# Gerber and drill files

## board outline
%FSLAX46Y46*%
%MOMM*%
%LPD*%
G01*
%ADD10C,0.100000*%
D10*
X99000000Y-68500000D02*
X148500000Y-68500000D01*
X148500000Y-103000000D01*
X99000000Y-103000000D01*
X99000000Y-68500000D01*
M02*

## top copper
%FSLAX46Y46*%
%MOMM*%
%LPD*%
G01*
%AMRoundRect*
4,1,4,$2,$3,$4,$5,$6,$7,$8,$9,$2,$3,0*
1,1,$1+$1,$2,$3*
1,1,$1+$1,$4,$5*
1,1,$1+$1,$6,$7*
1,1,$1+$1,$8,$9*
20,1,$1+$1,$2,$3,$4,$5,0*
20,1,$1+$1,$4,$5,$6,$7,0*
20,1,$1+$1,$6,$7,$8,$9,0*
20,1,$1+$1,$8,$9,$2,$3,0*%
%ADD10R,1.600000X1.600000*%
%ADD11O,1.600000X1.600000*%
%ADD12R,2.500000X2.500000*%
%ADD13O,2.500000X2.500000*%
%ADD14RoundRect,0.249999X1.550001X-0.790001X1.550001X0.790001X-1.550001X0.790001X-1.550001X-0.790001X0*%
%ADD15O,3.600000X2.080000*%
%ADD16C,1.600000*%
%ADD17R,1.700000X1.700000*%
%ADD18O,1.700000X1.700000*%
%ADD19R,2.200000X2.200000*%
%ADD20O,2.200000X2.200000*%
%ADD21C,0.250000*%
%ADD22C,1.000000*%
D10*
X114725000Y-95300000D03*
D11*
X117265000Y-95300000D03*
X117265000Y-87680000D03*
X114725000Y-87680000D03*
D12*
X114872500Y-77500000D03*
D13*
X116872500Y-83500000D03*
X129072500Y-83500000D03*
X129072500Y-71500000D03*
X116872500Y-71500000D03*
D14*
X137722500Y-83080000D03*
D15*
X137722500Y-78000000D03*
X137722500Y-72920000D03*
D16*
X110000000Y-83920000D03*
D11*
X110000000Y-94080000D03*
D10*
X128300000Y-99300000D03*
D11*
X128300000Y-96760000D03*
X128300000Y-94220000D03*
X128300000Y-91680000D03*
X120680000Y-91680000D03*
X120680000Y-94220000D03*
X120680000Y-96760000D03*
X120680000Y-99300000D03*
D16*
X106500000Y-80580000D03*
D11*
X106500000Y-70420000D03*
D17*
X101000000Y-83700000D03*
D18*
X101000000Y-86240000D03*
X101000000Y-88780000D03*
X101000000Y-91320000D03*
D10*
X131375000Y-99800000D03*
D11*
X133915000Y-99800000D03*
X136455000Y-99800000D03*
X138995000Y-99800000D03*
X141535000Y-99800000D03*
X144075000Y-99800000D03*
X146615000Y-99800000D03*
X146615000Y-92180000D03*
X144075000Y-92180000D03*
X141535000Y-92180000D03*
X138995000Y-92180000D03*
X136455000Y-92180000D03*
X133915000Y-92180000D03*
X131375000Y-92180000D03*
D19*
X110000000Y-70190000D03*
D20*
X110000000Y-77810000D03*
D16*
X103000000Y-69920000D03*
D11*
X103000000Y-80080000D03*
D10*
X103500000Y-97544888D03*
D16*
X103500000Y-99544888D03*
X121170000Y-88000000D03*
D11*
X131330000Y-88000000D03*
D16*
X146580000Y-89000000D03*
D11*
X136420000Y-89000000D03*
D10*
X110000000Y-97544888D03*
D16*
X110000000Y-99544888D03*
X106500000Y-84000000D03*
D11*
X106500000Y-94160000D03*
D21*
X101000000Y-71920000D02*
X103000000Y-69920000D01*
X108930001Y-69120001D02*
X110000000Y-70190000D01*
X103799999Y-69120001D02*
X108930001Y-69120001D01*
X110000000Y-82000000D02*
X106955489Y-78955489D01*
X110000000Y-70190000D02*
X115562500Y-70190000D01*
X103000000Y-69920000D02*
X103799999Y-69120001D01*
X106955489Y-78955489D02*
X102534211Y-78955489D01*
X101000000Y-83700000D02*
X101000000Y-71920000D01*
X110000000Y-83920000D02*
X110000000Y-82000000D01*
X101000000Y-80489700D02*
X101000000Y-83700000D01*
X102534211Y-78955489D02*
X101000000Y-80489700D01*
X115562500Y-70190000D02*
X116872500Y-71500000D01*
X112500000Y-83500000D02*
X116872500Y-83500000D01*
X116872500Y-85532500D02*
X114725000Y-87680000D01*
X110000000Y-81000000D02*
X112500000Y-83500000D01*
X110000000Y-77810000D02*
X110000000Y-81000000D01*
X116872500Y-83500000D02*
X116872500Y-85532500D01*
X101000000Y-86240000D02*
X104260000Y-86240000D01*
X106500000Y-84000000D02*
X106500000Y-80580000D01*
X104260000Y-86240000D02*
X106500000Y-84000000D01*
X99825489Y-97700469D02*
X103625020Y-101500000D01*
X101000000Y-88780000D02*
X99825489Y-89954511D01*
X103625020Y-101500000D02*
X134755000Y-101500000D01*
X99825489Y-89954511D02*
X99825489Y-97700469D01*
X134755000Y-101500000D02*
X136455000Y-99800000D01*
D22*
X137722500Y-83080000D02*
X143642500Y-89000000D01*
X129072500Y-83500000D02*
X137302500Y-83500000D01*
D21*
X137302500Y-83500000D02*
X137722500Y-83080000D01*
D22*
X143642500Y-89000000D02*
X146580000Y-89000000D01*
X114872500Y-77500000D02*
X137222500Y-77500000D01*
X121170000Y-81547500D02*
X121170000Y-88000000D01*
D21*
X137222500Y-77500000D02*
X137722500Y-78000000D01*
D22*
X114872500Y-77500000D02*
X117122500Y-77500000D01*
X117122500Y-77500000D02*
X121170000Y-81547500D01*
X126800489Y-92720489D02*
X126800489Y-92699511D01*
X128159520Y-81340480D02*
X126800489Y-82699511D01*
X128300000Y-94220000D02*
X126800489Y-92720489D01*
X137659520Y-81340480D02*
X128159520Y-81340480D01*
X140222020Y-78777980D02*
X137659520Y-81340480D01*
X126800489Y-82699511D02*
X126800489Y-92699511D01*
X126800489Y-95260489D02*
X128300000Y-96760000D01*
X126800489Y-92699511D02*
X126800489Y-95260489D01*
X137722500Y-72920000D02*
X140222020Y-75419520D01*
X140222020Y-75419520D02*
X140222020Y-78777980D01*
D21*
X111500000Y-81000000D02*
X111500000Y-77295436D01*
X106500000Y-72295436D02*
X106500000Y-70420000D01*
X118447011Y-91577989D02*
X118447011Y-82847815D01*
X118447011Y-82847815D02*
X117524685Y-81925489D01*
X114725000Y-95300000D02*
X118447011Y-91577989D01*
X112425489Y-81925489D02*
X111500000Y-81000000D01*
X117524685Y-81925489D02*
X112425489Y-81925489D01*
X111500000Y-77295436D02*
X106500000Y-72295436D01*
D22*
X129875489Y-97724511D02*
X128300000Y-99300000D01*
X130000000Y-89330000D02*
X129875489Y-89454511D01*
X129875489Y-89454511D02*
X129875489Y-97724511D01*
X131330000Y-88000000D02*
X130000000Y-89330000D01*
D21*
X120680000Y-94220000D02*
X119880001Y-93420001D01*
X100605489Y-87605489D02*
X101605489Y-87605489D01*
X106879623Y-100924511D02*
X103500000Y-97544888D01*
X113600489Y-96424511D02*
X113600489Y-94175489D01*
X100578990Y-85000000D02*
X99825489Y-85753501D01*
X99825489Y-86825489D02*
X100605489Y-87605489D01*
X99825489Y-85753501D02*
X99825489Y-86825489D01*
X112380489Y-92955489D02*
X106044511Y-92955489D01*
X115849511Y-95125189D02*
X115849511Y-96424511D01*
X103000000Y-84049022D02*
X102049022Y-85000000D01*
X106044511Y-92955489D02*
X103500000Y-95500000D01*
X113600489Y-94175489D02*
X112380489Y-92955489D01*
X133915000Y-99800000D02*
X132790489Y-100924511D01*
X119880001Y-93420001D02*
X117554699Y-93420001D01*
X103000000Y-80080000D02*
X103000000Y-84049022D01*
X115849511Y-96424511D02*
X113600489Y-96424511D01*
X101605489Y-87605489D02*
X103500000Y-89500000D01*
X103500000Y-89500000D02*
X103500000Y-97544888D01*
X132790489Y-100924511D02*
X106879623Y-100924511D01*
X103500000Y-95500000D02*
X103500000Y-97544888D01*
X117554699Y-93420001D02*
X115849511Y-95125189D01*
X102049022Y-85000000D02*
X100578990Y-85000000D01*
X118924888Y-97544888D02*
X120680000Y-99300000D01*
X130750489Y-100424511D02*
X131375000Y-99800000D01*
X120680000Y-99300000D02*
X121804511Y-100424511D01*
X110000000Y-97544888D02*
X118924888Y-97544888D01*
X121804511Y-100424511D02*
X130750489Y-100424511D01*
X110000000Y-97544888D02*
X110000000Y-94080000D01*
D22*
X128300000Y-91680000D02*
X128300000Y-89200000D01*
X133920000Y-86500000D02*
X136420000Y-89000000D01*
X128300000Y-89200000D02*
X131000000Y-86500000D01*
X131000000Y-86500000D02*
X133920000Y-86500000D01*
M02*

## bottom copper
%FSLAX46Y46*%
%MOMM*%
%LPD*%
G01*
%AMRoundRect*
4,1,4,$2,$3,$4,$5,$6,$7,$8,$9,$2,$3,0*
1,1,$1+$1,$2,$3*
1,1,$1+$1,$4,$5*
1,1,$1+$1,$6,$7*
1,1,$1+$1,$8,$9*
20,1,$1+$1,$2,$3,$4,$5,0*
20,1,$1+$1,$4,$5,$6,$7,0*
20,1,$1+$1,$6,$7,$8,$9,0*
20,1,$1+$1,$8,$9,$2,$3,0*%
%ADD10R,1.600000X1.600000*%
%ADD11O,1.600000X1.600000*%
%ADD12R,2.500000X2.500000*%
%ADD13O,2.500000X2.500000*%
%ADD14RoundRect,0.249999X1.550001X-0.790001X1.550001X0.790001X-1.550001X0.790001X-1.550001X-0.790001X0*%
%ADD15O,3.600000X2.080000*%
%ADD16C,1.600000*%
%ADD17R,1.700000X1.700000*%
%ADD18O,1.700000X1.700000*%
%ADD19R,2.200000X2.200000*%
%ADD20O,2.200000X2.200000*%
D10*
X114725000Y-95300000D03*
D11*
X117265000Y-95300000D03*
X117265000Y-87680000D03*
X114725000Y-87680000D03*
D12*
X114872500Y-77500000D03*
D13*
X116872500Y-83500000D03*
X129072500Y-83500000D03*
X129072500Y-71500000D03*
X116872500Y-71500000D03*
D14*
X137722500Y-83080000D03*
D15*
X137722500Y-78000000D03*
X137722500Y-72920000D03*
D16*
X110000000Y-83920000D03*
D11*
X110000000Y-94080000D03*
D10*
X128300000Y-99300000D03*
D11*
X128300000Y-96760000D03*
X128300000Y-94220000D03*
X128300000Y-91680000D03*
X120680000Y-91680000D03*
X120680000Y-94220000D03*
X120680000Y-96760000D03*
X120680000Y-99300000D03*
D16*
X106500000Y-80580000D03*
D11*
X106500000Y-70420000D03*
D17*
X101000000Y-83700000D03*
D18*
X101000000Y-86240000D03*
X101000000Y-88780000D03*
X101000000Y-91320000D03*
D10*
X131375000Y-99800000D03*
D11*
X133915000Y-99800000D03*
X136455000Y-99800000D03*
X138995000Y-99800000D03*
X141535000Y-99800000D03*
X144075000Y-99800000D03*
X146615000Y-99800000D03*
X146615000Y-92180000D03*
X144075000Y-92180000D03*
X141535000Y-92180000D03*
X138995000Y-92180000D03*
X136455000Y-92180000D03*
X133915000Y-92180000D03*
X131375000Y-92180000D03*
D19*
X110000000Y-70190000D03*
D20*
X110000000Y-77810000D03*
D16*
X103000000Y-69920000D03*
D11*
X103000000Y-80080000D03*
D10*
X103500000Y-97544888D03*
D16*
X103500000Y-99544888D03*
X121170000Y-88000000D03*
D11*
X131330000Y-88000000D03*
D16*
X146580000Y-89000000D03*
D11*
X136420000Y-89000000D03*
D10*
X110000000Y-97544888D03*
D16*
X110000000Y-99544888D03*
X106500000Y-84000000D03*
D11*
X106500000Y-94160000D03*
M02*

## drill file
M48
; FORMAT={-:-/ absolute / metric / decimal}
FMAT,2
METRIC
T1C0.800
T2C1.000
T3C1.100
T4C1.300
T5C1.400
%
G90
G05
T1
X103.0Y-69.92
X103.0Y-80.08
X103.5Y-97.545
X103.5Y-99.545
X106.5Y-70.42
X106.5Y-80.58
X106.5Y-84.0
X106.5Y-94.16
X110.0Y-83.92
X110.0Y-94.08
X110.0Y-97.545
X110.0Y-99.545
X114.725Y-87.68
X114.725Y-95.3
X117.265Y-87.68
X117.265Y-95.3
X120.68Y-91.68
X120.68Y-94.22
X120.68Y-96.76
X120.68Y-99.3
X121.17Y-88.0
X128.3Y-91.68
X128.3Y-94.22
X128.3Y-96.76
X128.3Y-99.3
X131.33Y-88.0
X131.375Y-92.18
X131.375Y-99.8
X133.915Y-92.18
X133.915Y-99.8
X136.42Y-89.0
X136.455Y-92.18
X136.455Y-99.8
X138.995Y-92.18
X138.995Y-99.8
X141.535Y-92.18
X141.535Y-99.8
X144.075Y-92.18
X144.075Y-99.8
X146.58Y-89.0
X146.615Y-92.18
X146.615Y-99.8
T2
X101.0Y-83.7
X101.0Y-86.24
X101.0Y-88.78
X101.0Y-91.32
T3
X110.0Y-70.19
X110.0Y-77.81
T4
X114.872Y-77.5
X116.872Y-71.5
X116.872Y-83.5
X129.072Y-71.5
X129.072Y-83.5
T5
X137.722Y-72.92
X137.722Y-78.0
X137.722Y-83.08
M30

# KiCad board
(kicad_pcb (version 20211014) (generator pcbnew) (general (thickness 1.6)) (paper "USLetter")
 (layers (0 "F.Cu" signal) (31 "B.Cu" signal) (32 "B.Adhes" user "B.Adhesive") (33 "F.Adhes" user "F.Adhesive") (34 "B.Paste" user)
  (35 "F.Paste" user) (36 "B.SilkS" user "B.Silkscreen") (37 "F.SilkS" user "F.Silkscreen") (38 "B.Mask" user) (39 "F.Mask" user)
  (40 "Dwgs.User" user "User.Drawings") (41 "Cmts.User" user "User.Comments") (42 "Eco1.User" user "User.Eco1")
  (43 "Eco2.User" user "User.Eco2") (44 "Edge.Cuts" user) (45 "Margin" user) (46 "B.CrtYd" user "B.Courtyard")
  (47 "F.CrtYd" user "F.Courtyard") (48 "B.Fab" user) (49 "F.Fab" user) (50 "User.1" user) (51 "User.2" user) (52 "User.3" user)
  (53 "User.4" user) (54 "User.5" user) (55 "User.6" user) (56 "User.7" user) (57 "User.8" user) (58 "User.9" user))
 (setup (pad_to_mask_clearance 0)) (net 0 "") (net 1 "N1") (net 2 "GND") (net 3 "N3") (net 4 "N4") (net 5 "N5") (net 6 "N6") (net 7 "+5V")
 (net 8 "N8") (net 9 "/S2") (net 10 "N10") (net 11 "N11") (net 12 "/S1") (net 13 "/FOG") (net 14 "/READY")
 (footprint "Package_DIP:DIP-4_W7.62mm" (layer "F.Cu") (at 114.725 95.3 90)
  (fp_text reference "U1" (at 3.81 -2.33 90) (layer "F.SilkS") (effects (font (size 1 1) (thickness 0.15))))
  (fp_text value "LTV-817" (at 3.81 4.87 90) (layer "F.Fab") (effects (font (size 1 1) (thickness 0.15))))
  (pad "1" thru_hole rect locked (at 0 0 90) (size 1.6 1.6) (drill 0.8) (layers *.Cu *.Mask) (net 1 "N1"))
  (pad "2" thru_hole oval locked (at 0 2.54 90) (size 1.6 1.6) (drill 0.8) (layers *.Cu *.Mask) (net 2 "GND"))
  (pad "3" thru_hole oval locked (at 7.62 2.54 90) (size 1.6 1.6) (drill 0.8) (layers *.Cu *.Mask) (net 2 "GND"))
  (pad "4" thru_hole oval locked (at 7.62 0 90) (size 1.6 1.6) (drill 0.8) (layers *.Cu *.Mask) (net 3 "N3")))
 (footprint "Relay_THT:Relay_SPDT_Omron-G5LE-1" (layer "F.Cu") (at 114.8725 77.5 90)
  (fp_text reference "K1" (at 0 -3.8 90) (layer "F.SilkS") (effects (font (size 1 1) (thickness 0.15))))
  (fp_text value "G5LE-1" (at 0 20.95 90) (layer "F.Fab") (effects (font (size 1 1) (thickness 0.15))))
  (pad "1" thru_hole rect locked (at 0 0 90) (size 2.5 2.5) (drill 1.3) (layers *.Cu *.Mask) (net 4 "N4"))
  (pad "2" thru_hole oval locked (at -6 2 90) (size 2.5 2.5) (drill 1.3) (layers *.Cu *.Mask) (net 3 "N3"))
  (pad "3" thru_hole oval locked (at -6 14.2 90) (size 2.5 2.5) (drill 1.3) (layers *.Cu *.Mask) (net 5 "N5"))
  (pad "4" thru_hole oval locked (at 6 14.2 90) (size 2.5 2.5) (drill 1.3) (layers *.Cu *.Mask) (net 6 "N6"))
  (pad "5" thru_hole oval locked (at 6 2 90) (size 2.5 2.5) (drill 1.3) (layers *.Cu *.Mask) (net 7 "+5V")))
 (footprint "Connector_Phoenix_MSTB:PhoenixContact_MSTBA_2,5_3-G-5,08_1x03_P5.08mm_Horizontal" (layer "F.Cu") (at 137.7225 83.08 90)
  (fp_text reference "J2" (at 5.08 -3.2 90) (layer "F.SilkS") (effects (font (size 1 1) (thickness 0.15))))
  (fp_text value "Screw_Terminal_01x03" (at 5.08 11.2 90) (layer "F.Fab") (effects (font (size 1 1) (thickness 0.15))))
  (pad "1" thru_hole roundrect locked (at 0 0 90) (size 2.08 3.6) (drill 1.4) (layers *.Cu *.Mask) (roundrect_rratio 0.120192) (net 5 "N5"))
  (pad "2" thru_hole oval locked (at 5.08 0 90) (size 2.08 3.6) (drill 1.4) (layers *.Cu *.Mask) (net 4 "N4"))
  (pad "3" thru_hole oval locked (at 10.16 0 90) (size 2.08 3.6) (drill 1.4) (layers *.Cu *.Mask) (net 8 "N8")))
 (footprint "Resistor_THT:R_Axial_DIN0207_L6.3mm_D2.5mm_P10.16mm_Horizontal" (layer "F.Cu") (at 110 83.92 -90)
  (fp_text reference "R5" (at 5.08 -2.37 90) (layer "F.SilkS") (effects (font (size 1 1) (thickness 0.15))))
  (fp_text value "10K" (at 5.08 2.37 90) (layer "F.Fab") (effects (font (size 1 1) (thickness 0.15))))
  (pad "1" thru_hole circle locked (at 0 0 270) (size 1.6 1.6) (drill 0.8) (layers *.Cu *.Mask) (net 7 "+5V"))
  (pad "2" thru_hole oval locked (at 10.16 0 270) (size 1.6 1.6) (drill 0.8) (layers *.Cu *.Mask) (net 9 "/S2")))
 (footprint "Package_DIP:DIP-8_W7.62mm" (layer "F.Cu") (at 128.3 99.3 180)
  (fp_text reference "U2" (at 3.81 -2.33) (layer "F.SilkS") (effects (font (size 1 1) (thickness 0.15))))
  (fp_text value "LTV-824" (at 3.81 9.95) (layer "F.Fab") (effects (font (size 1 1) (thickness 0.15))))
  (pad "1" thru_hole rect locked (at 0 0 180) (size 1.6 1.6) (drill 0.8) (layers *.Cu *.Mask) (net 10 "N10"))
  (pad "2" thru_hole oval locked (at 0 2.54 180) (size 1.6 1.6) (drill 0.8) (layers *.Cu *.Mask) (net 8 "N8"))
  (pad "3" thru_hole oval locked (at 0 5.08 180) (size 1.6 1.6) (drill 0.8) (layers *.Cu *.Mask) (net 8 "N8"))
  (pad "4" thru_hole oval locked (at 0 7.62 180) (size 1.6 1.6) (drill 0.8) (layers *.Cu *.Mask) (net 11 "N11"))
  (pad "5" thru_hole oval locked (at 7.62 7.62 180) (size 1.6 1.6) (drill 0.8) (layers *.Cu *.Mask) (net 2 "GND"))
  (pad "6" thru_hole oval locked (at 7.62 5.08 180) (size 1.6 1.6) (drill 0.8) (layers *.Cu *.Mask) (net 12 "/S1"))
  (pad "7" thru_hole oval locked (at 7.62 2.54 180) (size 1.6 1.6) (drill 0.8) (layers *.Cu *.Mask) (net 2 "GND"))
  (pad "8" thru_hole oval locked (at 7.62 0 180) (size 1.6 1.6) (drill 0.8) (layers *.Cu *.Mask) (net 9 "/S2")))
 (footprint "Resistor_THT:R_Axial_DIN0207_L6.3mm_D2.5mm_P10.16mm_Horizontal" (layer "F.Cu") (at 106.5 80.58 90)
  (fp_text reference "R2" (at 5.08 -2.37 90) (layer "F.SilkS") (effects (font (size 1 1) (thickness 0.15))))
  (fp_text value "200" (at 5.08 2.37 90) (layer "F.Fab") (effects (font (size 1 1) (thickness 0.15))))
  (pad "1" thru_hole circle locked (at 0 0 90) (size 1.6 1.6) (drill 0.8) (layers *.Cu *.Mask) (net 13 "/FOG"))
  (pad "2" thru_hole oval locked (at 10.16 0 90) (size 1.6 1.6) (drill 0.8) (layers *.Cu *.Mask) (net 1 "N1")))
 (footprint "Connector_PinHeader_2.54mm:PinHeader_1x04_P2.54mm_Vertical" (layer "F.Cu") (at 101 83.7)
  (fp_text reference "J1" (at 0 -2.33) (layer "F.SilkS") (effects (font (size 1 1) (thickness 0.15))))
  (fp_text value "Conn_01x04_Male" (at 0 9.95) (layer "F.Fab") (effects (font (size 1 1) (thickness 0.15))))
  (pad "1" thru_hole rect locked (at 0 0) (size 1.7 1.7) (drill 1) (layers *.Cu *.Mask) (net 7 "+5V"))
  (pad "2" thru_hole oval locked (at 0 2.54) (size 1.7 1.7) (drill 1) (layers *.Cu *.Mask) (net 13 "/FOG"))
  (pad "3" thru_hole oval locked (at 0 5.08) (size 1.7 1.7) (drill 1) (layers *.Cu *.Mask) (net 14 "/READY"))
  (pad "4" thru_hole oval locked (at 0 7.62) (size 1.7 1.7) (drill 1) (layers *.Cu *.Mask) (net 2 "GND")))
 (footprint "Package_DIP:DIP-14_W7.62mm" (layer "F.Cu") (at 131.375 99.8 90)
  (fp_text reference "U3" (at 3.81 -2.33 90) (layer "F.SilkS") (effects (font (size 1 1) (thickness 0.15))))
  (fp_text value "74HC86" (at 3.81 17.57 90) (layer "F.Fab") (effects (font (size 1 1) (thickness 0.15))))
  (pad "1" thru_hole rect locked (at 0 0 90) (size 1.6 1.6) (drill 0.8) (layers *.Cu *.Mask) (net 9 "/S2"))
  (pad "2" thru_hole oval locked (at 0 2.54 90) (size 1.6 1.6) (drill 0.8) (layers *.Cu *.Mask) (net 12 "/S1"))
  (pad "3" thru_hole oval locked (at 0 5.08 90) (size 1.6 1.6) (drill 0.8) (layers *.Cu *.Mask) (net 14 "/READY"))
  (pad "4" thru_hole oval locked (at 0 7.62 90) (size 1.6 1.6) (drill 0.8) (layers *.Cu *.Mask))
  (pad "5" thru_hole oval locked (at 0 10.16 90) (size 1.6 1.6) (drill 0.8) (layers *.Cu *.Mask))
  (pad "6" thru_hole oval locked (at 0 12.7 90) (size 1.6 1.6) (drill 0.8) (layers *.Cu *.Mask))
  (pad "7" thru_hole oval locked (at 0 15.24 90) (size 1.6 1.6) (drill 0.8) (layers *.Cu *.Mask))
  (pad "8" thru_hole oval locked (at 7.62 15.24 90) (size 1.6 1.6) (drill 0.8) (layers *.Cu *.Mask))
  (pad "9" thru_hole oval locked (at 7.62 12.7 90) (size 1.6 1.6) (drill 0.8) (layers *.Cu *.Mask))
  (pad "10" thru_hole oval locked (at 7.62 10.16 90) (size 1.6 1.6) (drill 0.8) (layers *.Cu *.Mask))
  (pad "11" thru_hole oval locked (at 7.62 7.62 90) (size 1.6 1.6) (drill 0.8) (layers *.Cu *.Mask))
  (pad "12" thru_hole oval locked (at 7.62 5.08 90) (size 1.6 1.6) (drill 0.8) (layers *.Cu *.Mask))
  (pad "13" thru_hole oval locked (at 7.62 2.54 90) (size 1.6 1.6) (drill 0.8) (layers *.Cu *.Mask))
  (pad "14" thru_hole oval locked (at 7.62 0 90) (size 1.6 1.6) (drill 0.8) (layers *.Cu *.Mask)))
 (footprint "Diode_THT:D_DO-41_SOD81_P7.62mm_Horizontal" (layer "F.Cu") (at 110 70.19 -90)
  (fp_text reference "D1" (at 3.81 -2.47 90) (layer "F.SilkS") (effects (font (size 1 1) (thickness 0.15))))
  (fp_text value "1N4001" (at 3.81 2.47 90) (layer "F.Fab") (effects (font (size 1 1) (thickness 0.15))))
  (pad "1" thru_hole rect locked (at 0 0 270) (size 2.2 2.2) (drill 1.1) (layers *.Cu *.Mask) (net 7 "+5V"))
  (pad "2" thru_hole oval locked (at 7.62 0 270) (size 2.2 2.2) (drill 1.1) (layers *.Cu *.Mask) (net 3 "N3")))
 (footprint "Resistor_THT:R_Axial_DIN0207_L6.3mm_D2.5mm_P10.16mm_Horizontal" (layer "F.Cu") (at 103 69.92 -90)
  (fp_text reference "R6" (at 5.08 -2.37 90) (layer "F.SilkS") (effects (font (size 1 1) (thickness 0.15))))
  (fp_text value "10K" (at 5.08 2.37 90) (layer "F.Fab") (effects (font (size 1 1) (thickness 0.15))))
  (pad "1" thru_hole circle locked (at 0 0 270) (size 1.6 1.6) (drill 0.8) (layers *.Cu *.Mask) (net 7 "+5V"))
  (pad "2" thru_hole oval locked (at 10.16 0 270) (size 1.6 1.6) (drill 0.8) (layers *.Cu *.Mask) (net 12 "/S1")))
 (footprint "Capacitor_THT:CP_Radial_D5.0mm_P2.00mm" (layer "F.Cu") (at 103.5 97.544888 -90)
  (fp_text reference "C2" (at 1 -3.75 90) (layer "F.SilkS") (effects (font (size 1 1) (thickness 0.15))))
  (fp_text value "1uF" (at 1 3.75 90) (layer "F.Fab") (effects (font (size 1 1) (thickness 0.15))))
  (pad "1" thru_hole rect locked (at 0 0 270) (size 1.6 1.6) (drill 0.8) (layers *.Cu *.Mask) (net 12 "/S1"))
  (pad "2" thru_hole circle locked (at 2 0 270) (size 1.6 1.6) (drill 0.8) (layers *.Cu *.Mask) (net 2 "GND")))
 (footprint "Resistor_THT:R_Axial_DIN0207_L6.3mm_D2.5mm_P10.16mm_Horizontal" (layer "F.Cu") (at 121.17 88)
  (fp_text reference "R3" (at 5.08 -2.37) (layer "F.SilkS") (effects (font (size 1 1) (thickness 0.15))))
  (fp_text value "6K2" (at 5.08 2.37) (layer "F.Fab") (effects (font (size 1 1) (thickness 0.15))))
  (pad "1" thru_hole circle locked (at 0 0) (size 1.6 1.6) (drill 0.8) (layers *.Cu *.Mask) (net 4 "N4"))
  (pad "2" thru_hole oval locked (at 10.16 0) (size 1.6 1.6) (drill 0.8) (layers *.Cu *.Mask) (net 10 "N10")))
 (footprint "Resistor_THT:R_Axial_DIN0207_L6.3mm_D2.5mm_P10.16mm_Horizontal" (layer "F.Cu") (at 146.58 89 180)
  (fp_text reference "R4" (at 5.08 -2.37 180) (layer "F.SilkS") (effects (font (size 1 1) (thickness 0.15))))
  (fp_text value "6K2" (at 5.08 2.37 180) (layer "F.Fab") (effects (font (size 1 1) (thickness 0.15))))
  (pad "1" thru_hole circle locked (at 0 0 180) (size 1.6 1.6) (drill 0.8) (layers *.Cu *.Mask) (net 5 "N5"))
  (pad "2" thru_hole oval locked (at 10.16 0 180) (size 1.6 1.6) (drill 0.8) (layers *.Cu *.Mask) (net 11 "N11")))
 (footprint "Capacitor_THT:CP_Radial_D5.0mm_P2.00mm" (layer "F.Cu") (at 110 97.544888 -90)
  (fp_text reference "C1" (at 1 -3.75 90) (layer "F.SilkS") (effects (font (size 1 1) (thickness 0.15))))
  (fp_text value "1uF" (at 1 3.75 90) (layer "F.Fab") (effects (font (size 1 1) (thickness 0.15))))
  (pad "1" thru_hole rect locked (at 0 0 270) (size 1.6 1.6) (drill 0.8) (layers *.Cu *.Mask) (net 9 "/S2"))
  (pad "2" thru_hole circle locked (at 2 0 270) (size 1.6 1.6) (drill 0.8) (layers *.Cu *.Mask) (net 2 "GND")))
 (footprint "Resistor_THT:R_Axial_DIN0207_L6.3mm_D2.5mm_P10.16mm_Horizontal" (layer "F.Cu") (at 106.5 84 -90)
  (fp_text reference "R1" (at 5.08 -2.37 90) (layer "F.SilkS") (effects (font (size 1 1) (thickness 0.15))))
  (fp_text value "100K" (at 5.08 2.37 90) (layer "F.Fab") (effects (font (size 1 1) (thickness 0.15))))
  (pad "1" thru_hole circle locked (at 0 0 270) (size 1.6 1.6) (drill 0.8) (layers *.Cu *.Mask) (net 13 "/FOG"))
  (pad "2" thru_hole oval locked (at 10.16 0 270) (size 1.6 1.6) (drill 0.8) (layers *.Cu *.Mask) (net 2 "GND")))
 (gr_rect (start 99 68.5) (end 148.5 103) (layer "Edge.Cuts") (width 0.1) (fill none))
 (segment (start 101 71.92) (end 103 69.92) (width 0.25) (layer "F.Cu") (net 7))
 (segment (start 108.930001 69.120001) (end 110 70.19) (width 0.25) (layer "F.Cu") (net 7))
 (segment (start 103.799999 69.120001) (end 108.930001 69.120001) (width 0.25) (layer "F.Cu") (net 7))
 (segment (start 110 82) (end 106.955489 78.955489) (width 0.25) (layer "F.Cu") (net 7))
 (segment (start 110 70.19) (end 115.5625 70.19) (width 0.25) (layer "F.Cu") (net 7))
 (segment (start 103 69.92) (end 103.799999 69.120001) (width 0.25) (layer "F.Cu") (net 7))
 (segment (start 106.955489 78.955489) (end 102.534211 78.955489) (width 0.25) (layer "F.Cu") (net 7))
 (segment (start 101 83.7) (end 101 71.92) (width 0.25) (layer "F.Cu") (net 7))
 (segment (start 110 83.92) (end 110 82) (width 0.25) (layer "F.Cu") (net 7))
 (segment (start 101 80.4897) (end 101 83.7) (width 0.25) (layer "F.Cu") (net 7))
 (segment (start 102.534211 78.955489) (end 101 80.4897) (width 0.25) (layer "F.Cu") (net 7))
 (segment (start 115.5625 70.19) (end 116.8725 71.5) (width 0.25) (layer "F.Cu") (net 7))
 (segment (start 112.5 83.5) (end 116.8725 83.5) (width 0.25) (layer "F.Cu") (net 3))
 (segment (start 116.8725 85.5325) (end 114.725 87.68) (width 0.25) (layer "F.Cu") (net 3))
 (segment (start 110 81) (end 112.5 83.5) (width 0.25) (layer "F.Cu") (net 3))
 (segment (start 110 77.81) (end 110 81) (width 0.25) (layer "F.Cu") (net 3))
 (segment (start 116.8725 83.5) (end 116.8725 85.5325) (width 0.25) (layer "F.Cu") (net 3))
 (segment (start 101 86.24) (end 104.26 86.24) (width 0.25) (layer "F.Cu") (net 13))
 (segment (start 106.5 84) (end 106.5 80.58) (width 0.25) (layer "F.Cu") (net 13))
 (segment (start 104.26 86.24) (end 106.5 84) (width 0.25) (layer "F.Cu") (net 13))
 (segment (start 99.825489 97.700469) (end 103.62502 101.5) (width 0.25) (layer "F.Cu") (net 14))
 (segment (start 101 88.78) (end 99.825489 89.954511) (width 0.25) (layer "F.Cu") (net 14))
 (segment (start 103.62502 101.5) (end 134.755 101.5) (width 0.25) (layer "F.Cu") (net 14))
 (segment (start 99.825489 89.954511) (end 99.825489 97.700469) (width 0.25) (layer "F.Cu") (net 14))
 (segment (start 134.755 101.5) (end 136.455 99.8) (width 0.25) (layer "F.Cu") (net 14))
 (segment (start 137.7225 83.08) (end 143.6425 89) (width 1) (layer "F.Cu") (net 5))
 (segment (start 129.0725 83.5) (end 137.3025 83.5) (width 1) (layer "F.Cu") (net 5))
 (segment (start 137.3025 83.5) (end 137.7225 83.08) (width 0.25) (layer "F.Cu") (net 5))
 (segment (start 143.6425 89) (end 146.58 89) (width 1) (layer "F.Cu") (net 5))
 (segment (start 114.8725 77.5) (end 137.2225 77.5) (width 1) (layer "F.Cu") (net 4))
 (segment (start 121.17 81.5475) (end 121.17 88) (width 1) (layer "F.Cu") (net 4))
 (segment (start 137.2225 77.5) (end 137.7225 78) (width 0.25) (layer "F.Cu") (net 4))
 (segment (start 114.8725 77.5) (end 117.1225 77.5) (width 1) (layer "F.Cu") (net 4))
 (segment (start 117.1225 77.5) (end 121.17 81.5475) (width 1) (layer "F.Cu") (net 4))
 (segment (start 126.800489 92.720489) (end 126.800489 92.699511) (width 1) (layer "F.Cu") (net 8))
 (segment (start 128.15952 81.34048) (end 126.800489 82.699511) (width 1) (layer "F.Cu") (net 8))
 (segment (start 128.3 94.22) (end 126.800489 92.720489) (width 1) (layer "F.Cu") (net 8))
 (segment (start 137.65952 81.34048) (end 128.15952 81.34048) (width 1) (layer "F.Cu") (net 8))
 (segment (start 140.22202 78.77798) (end 137.65952 81.34048) (width 1) (layer "F.Cu") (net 8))
 (segment (start 126.800489 82.699511) (end 126.800489 92.699511) (width 1) (layer "F.Cu") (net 8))
 (segment (start 126.800489 95.260489) (end 128.3 96.76) (width 1) (layer "F.Cu") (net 8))
 (segment (start 126.800489 92.699511) (end 126.800489 95.260489) (width 1) (layer "F.Cu") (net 8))
 (segment (start 137.7225 72.92) (end 140.22202 75.41952) (width 1) (layer "F.Cu") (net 8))
 (segment (start 140.22202 75.41952) (end 140.22202 78.77798) (width 1) (layer "F.Cu") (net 8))
 (segment (start 111.5 81) (end 111.5 77.295436) (width 0.25) (layer "F.Cu") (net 1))
 (segment (start 106.5 72.295436) (end 106.5 70.42) (width 0.25) (layer "F.Cu") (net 1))
 (segment (start 118.447011 91.577989) (end 118.447011 82.847815) (width 0.25) (layer "F.Cu") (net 1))
 (segment (start 118.447011 82.847815) (end 117.524685 81.925489) (width 0.25) (layer "F.Cu") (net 1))
 (segment (start 114.725 95.3) (end 118.447011 91.577989) (width 0.25) (layer "F.Cu") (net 1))
 (segment (start 112.425489 81.925489) (end 111.5 81) (width 0.25) (layer "F.Cu") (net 1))
 (segment (start 117.524685 81.925489) (end 112.425489 81.925489) (width 0.25) (layer "F.Cu") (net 1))
 (segment (start 111.5 77.295436) (end 106.5 72.295436) (width 0.25) (layer "F.Cu") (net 1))
 (segment (start 129.875489 97.724511) (end 128.3 99.3) (width 1) (layer "F.Cu") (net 10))
 (segment (start 130 89.33) (end 129.875489 89.454511) (width 1) (layer "F.Cu") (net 10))
 (segment (start 129.875489 89.454511) (end 129.875489 97.724511) (width 1) (layer "F.Cu") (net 10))
 (segment (start 131.33 88) (end 130 89.33) (width 1) (layer "F.Cu") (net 10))
 (segment (start 120.68 94.22) (end 119.880001 93.420001) (width 0.25) (layer "F.Cu") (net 12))
 (segment (start 100.605489 87.605489) (end 101.605489 87.605489) (width 0.25) (layer "F.Cu") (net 12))
 (segment (start 106.879623 100.924511) (end 103.5 97.544888) (width 0.25) (layer "F.Cu") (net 12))
 (segment (start 113.600489 96.424511) (end 113.600489 94.175489) (width 0.25) (layer "F.Cu") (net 12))
 (segment (start 100.57899 85) (end 99.825489 85.753501) (width 0.25) (layer "F.Cu") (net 12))
 (segment (start 99.825489 86.825489) (end 100.605489 87.605489) (width 0.25) (layer "F.Cu") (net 12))
 (segment (start 99.825489 85.753501) (end 99.825489 86.825489) (width 0.25) (layer "F.Cu") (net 12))
 (segment (start 112.380489 92.955489) (end 106.044511 92.955489) (width 0.25) (layer "F.Cu") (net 12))
 (segment (start 115.849511 95.125189) (end 115.849511 96.424511) (width 0.25) (layer "F.Cu") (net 12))
 (segment (start 103 84.049022) (end 102.049022 85) (width 0.25) (layer "F.Cu") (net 12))
 (segment (start 106.044511 92.955489) (end 103.5 95.5) (width 0.25) (layer "F.Cu") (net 12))
 (segment (start 113.600489 94.175489) (end 112.380489 92.955489) (width 0.25) (layer "F.Cu") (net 12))
 (segment (start 133.915 99.8) (end 132.790489 100.924511) (width 0.25) (layer "F.Cu") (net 12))
 (segment (start 119.880001 93.420001) (end 117.554699 93.420001) (width 0.25) (layer "F.Cu") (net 12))
 (segment (start 103 80.08) (end 103 84.049022) (width 0.25) (layer "F.Cu") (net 12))
 (segment (start 115.849511 96.424511) (end 113.600489 96.424511) (width 0.25) (layer "F.Cu") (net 12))
 (segment (start 101.605489 87.605489) (end 103.5 89.5) (width 0.25) (layer "F.Cu") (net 12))
 (segment (start 103.5 89.5) (end 103.5 97.544888) (width 0.25) (layer "F.Cu") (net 12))
 (segment (start 132.790489 100.924511) (end 106.879623 100.924511) (width 0.25) (layer "F.Cu") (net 12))
 (segment (start 103.5 95.5) (end 103.5 97.544888) (width 0.25) (layer "F.Cu") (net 12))
 (segment (start 117.554699 93.420001) (end 115.849511 95.125189) (width 0.25) (layer "F.Cu") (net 12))
 (segment (start 102.049022 85) (end 100.57899 85) (width 0.25) (layer "F.Cu") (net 12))
 (segment (start 118.924888 97.544888) (end 120.68 99.3) (width 0.25) (layer "F.Cu") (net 9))
 (segment (start 130.750489 100.424511) (end 131.375 99.8) (width 0.25) (layer "F.Cu") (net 9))
 (segment (start 120.68 99.3) (end 121.804511 100.424511) (width 0.25) (layer "F.Cu") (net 9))
 (segment (start 110 97.544888) (end 118.924888 97.544888) (width 0.25) (layer "F.Cu") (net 9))
 (segment (start 121.804511 100.424511) (end 130.750489 100.424511) (width 0.25) (layer "F.Cu") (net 9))
 (segment (start 110 97.544888) (end 110 94.08) (width 0.25) (layer "F.Cu") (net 9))
 (segment (start 128.3 91.68) (end 128.3 89.2) (width 1) (layer "F.Cu") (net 11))
 (segment (start 133.92 86.5) (end 136.42 89) (width 1) (layer "F.Cu") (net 11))
 (segment (start 128.3 89.2) (end 131 86.5) (width 1) (layer "F.Cu") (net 11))
 (segment (start 131 86.5) (end 133.92 86.5) (width 1) (layer "F.Cu") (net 11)))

